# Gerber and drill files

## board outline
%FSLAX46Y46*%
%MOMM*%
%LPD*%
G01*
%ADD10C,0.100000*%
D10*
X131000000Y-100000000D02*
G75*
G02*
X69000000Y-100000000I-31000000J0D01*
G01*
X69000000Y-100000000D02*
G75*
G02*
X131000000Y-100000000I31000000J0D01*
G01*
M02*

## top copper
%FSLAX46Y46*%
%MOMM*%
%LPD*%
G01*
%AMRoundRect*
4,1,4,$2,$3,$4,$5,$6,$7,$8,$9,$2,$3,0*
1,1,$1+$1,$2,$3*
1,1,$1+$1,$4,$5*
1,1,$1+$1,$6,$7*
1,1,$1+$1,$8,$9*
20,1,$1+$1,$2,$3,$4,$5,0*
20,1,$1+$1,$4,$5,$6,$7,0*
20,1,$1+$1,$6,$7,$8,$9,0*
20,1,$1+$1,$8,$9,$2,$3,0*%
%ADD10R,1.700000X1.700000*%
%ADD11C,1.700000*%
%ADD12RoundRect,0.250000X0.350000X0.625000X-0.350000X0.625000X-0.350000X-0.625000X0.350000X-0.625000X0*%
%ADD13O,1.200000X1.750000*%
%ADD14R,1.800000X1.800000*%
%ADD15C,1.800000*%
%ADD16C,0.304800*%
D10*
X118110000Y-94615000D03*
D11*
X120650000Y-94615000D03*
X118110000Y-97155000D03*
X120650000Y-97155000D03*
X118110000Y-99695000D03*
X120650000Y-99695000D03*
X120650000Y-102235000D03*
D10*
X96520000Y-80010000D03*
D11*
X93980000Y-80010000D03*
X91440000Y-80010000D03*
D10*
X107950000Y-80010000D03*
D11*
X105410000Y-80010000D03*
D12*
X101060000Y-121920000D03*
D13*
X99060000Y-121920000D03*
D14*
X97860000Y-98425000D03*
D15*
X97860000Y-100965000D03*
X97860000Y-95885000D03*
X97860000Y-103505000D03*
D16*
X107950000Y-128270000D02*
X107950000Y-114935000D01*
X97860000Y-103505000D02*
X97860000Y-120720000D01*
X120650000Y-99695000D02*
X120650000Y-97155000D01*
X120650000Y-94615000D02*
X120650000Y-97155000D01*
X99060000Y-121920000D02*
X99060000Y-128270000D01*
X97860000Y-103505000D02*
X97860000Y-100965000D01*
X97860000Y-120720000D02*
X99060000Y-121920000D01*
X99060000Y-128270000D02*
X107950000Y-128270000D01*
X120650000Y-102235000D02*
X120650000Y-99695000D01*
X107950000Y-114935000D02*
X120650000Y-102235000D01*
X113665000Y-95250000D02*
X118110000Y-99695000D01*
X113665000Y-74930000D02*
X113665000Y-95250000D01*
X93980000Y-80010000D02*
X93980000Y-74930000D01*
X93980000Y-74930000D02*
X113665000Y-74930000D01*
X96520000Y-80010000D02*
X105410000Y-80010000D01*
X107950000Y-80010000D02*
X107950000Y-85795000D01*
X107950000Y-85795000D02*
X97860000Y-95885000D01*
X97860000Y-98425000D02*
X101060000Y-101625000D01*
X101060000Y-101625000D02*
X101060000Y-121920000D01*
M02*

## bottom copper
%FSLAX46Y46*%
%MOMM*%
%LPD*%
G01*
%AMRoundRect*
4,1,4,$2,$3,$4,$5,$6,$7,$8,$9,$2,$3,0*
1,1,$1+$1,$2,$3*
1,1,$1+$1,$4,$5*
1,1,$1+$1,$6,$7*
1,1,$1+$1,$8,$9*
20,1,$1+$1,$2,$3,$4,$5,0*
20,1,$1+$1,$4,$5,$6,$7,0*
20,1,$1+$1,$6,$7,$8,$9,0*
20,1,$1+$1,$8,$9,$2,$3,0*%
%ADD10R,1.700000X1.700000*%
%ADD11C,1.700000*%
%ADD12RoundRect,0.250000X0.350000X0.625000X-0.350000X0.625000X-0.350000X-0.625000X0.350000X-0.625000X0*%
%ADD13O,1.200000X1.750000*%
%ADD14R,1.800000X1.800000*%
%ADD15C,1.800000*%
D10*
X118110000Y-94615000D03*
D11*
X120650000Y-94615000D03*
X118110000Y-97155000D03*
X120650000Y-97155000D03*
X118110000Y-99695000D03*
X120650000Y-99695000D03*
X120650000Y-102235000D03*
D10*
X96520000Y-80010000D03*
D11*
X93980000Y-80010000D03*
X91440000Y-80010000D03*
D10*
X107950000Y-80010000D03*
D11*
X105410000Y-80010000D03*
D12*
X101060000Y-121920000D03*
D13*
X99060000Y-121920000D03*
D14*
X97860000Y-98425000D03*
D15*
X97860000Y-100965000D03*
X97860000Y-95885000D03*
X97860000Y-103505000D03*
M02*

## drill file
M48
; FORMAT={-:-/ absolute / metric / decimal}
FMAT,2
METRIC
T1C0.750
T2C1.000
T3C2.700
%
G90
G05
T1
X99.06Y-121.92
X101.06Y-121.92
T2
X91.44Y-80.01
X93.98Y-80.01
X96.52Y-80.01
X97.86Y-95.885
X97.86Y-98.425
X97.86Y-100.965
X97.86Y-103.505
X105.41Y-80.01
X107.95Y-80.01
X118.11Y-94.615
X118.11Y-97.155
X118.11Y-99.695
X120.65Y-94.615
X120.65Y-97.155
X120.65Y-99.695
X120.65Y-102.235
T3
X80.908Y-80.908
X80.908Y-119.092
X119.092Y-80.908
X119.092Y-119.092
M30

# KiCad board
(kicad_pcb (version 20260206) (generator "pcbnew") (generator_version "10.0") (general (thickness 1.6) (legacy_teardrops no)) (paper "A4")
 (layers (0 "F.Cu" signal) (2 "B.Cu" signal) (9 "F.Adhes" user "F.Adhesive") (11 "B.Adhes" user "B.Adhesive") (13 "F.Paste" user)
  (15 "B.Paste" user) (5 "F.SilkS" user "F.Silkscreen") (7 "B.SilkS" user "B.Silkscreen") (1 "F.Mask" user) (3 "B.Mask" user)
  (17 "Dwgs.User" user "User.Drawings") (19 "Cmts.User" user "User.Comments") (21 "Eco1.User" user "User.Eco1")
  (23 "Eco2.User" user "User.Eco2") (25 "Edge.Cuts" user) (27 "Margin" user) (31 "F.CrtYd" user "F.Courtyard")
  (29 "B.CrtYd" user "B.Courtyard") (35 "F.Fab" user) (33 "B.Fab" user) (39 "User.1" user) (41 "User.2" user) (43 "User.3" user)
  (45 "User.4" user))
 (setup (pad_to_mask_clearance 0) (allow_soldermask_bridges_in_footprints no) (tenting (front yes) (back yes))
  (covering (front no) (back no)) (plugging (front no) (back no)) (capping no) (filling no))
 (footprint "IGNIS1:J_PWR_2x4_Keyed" (layer "F.Cu") (at 119.38 98.425)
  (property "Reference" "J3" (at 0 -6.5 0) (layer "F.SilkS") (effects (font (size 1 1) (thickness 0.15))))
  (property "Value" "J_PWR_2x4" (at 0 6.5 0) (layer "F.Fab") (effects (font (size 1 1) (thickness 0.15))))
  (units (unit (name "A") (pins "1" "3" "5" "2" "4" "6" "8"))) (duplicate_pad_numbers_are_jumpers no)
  (pad "1" thru_hole rect (at -1.27 -3.81) (size 1.7 1.7) (drill 1) (layers "*.Cu" "*.Mask") (remove_unused_layers no)
   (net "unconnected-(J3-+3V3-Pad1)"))
  (pad "2" thru_hole circle (at 1.27 -3.81) (size 1.7 1.7) (drill 1) (layers "*.Cu" "*.Mask") (remove_unused_layers no) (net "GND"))
  (pad "3" thru_hole circle (at -1.27 -1.27) (size 1.7 1.7) (drill 1) (layers "*.Cu" "*.Mask") (remove_unused_layers no)
   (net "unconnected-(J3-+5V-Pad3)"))
  (pad "4" thru_hole circle (at 1.27 -1.27) (size 1.7 1.7) (drill 1) (layers "*.Cu" "*.Mask") (remove_unused_layers no) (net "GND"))
  (pad "5" thru_hole circle (at -1.27 1.27) (size 1.7 1.7) (drill 1) (layers "*.Cu" "*.Mask") (remove_unused_layers no) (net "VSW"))
  (pad "6" thru_hole circle (at 1.27 1.27) (size 1.7 1.7) (drill 1) (layers "*.Cu" "*.Mask") (remove_unused_layers no) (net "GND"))
  (pad "8" thru_hole circle (at 1.27 3.81) (size 1.7 1.7) (drill 1) (layers "*.Cu" "*.Mask") (remove_unused_layers no) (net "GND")))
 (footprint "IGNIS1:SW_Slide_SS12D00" (layer "F.Cu") (at 93.98 80.01 180)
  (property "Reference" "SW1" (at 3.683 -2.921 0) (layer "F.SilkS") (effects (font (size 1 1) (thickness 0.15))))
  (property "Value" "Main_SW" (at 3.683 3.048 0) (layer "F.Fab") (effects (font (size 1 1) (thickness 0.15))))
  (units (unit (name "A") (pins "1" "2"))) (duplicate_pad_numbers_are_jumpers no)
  (pad "1" thru_hole rect (at -2.54 0 180) (size 1.7 1.7) (drill 1) (layers "*.Cu" "*.Mask") (remove_unused_layers no) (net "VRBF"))
  (pad "2" thru_hole circle (at 0 0 180) (size 1.7 1.7) (drill 1) (layers "*.Cu" "*.Mask") (remove_unused_layers no) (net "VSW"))
  (pad "3" thru_hole circle (at 2.54 0 180) (size 1.7 1.7) (drill 1) (layers "*.Cu" "*.Mask") (remove_unused_layers no)))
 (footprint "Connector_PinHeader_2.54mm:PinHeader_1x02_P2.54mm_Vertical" (layer "F.Cu") (at 107.95 80.01 -90)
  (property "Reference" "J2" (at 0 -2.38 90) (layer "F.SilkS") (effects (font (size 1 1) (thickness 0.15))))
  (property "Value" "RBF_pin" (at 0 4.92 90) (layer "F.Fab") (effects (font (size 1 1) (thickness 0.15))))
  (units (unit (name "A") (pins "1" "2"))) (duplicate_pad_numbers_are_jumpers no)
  (pad "1" thru_hole rect (at 0 0 270) (size 1.7 1.7) (drill 1) (layers "*.Cu" "*.Mask") (remove_unused_layers no) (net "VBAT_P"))
  (pad "2" thru_hole circle (at 0 2.54 270) (size 1.7 1.7) (drill 1) (layers "*.Cu" "*.Mask") (remove_unused_layers no) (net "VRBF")))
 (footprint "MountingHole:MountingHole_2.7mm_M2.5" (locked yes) (layer "F.Cu") (at 119.092 80.908)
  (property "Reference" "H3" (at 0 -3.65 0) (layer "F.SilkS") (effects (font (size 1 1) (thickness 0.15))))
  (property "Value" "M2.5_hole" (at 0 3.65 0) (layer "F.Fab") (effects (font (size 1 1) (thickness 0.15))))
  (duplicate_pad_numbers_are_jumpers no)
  (pad "" np_thru_hole circle (at 0 0) (size 2.7 2.7) (drill 2.7) (layers "*.Cu" "*.Mask")))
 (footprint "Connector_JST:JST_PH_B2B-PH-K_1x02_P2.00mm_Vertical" (layer "F.Cu") (at 101.06 121.92 180)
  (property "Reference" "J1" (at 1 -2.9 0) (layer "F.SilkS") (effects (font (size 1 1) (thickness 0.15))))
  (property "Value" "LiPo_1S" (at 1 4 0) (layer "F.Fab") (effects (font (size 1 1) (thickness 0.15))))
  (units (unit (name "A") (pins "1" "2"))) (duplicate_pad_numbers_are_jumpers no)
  (pad "1" thru_hole roundrect (at 0 0 180) (size 1.2 1.75) (drill 0.75) (layers "*.Cu" "*.Mask") (remove_unused_layers no)
   (roundrect_rratio 0.208333) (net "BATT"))
  (pad "2" thru_hole oval (at 2 0 180) (size 1.2 1.75) (drill 0.75) (layers "*.Cu" "*.Mask") (remove_unused_layers no) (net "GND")))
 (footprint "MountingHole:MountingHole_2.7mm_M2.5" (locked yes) (layer "F.Cu") (at 119.092 119.092)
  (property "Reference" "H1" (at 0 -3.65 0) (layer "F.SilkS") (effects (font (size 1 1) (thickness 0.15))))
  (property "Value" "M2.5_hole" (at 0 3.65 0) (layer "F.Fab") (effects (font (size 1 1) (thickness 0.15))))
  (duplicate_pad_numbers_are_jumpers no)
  (pad "" np_thru_hole circle (at 0 0) (size 2.7 2.7) (drill 2.7) (layers "*.Cu" "*.Mask")))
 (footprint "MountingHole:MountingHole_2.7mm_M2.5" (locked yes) (layer "F.Cu") (at 80.908 80.908)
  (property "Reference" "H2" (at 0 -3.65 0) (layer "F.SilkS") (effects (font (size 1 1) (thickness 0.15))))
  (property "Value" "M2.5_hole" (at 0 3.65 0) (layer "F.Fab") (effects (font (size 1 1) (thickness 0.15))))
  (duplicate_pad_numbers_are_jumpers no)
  (pad "" np_thru_hole circle (at 0 0) (size 2.7 2.7) (drill 2.7) (layers "*.Cu" "*.Mask")))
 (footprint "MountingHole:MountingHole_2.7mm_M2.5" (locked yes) (layer "F.Cu") (at 80.908 119.092)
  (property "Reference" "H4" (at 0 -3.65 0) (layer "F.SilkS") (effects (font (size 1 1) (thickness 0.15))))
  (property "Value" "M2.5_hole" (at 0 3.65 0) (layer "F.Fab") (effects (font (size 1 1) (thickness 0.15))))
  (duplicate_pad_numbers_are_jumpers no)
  (pad "" np_thru_hole circle (at 0 0) (size 2.7 2.7) (drill 2.7) (layers "*.Cu" "*.Mask")))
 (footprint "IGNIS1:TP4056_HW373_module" (layer "F.Cu") (at 86.36 99.695)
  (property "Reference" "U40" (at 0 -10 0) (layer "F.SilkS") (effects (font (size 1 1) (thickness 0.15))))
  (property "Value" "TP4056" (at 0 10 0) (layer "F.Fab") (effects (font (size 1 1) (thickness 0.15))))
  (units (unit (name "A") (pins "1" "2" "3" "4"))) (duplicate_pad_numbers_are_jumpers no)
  (pad "1" thru_hole rect (at 11.5 -1.27) (size 1.8 1.8) (drill 1) (layers "*.Cu" "*.Mask") (remove_unused_layers no) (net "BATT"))
  (pad "2" thru_hole circle (at 11.5 1.27) (size 1.8 1.8) (drill 1) (layers "*.Cu" "*.Mask") (remove_unused_layers no) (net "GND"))
  (pad "3" thru_hole circle (at 11.5 -3.81) (size 1.8 1.8) (drill 1) (layers "*.Cu" "*.Mask") (remove_unused_layers no) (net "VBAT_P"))
  (pad "4" thru_hole circle (at 11.5 3.81) (size 1.8 1.8) (drill 1) (layers "*.Cu" "*.Mask") (remove_unused_layers no) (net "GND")))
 (gr_circle (center 100 100) (end 131 100) (stroke (width 0.1) (type solid)) (fill no) (locked yes) (layer "Edge.Cuts"))
 (segment (start 107.95 128.27) (end 107.95 114.935) (width 0.3048) (layer "F.Cu") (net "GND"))
 (segment (start 97.86 103.505) (end 97.86 120.72) (width 0.3048) (layer "F.Cu") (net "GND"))
 (segment (start 120.65 99.695) (end 120.65 97.155) (width 0.3048) (layer "F.Cu") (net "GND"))
 (segment (start 120.65 94.615) (end 120.65 97.155) (width 0.3048) (layer "F.Cu") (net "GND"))
 (segment (start 99.06 121.92) (end 99.06 128.27) (width 0.3048) (layer "F.Cu") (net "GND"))
 (segment (start 97.86 103.505) (end 97.86 100.965) (width 0.3048) (layer "F.Cu") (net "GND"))
 (segment (start 97.86 120.72) (end 99.06 121.92) (width 0.3048) (layer "F.Cu") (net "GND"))
 (segment (start 99.06 128.27) (end 107.95 128.27) (width 0.3048) (layer "F.Cu") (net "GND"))
 (segment (start 120.65 102.235) (end 120.65 99.695) (width 0.3048) (layer "F.Cu") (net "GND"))
 (segment (start 107.95 114.935) (end 120.65 102.235) (width 0.3048) (layer "F.Cu") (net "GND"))
 (segment (start 113.665 95.25) (end 118.11 99.695) (width 0.3048) (layer "F.Cu") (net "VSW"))
 (segment (start 113.665 74.93) (end 113.665 95.25) (width 0.3048) (layer "F.Cu") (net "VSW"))
 (segment (start 93.98 80.01) (end 93.98 74.93) (width 0.3048) (layer "F.Cu") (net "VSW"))
 (segment (start 93.98 74.93) (end 113.665 74.93) (width 0.3048) (layer "F.Cu") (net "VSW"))
 (segment (start 96.52 80.01) (end 105.41 80.01) (width 0.3048) (layer "F.Cu") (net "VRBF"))
 (segment (start 107.95 80.01) (end 107.95 85.795) (width 0.3048) (layer "F.Cu") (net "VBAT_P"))
 (segment (start 107.95 85.795) (end 97.86 95.885) (width 0.3048) (layer "F.Cu") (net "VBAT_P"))
 (segment (start 97.86 98.425) (end 101.06 101.625) (width 0.3048) (layer "F.Cu") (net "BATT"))
 (segment (start 101.06 101.625) (end 101.06 121.92) (width 0.3048) (layer "F.Cu") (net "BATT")))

